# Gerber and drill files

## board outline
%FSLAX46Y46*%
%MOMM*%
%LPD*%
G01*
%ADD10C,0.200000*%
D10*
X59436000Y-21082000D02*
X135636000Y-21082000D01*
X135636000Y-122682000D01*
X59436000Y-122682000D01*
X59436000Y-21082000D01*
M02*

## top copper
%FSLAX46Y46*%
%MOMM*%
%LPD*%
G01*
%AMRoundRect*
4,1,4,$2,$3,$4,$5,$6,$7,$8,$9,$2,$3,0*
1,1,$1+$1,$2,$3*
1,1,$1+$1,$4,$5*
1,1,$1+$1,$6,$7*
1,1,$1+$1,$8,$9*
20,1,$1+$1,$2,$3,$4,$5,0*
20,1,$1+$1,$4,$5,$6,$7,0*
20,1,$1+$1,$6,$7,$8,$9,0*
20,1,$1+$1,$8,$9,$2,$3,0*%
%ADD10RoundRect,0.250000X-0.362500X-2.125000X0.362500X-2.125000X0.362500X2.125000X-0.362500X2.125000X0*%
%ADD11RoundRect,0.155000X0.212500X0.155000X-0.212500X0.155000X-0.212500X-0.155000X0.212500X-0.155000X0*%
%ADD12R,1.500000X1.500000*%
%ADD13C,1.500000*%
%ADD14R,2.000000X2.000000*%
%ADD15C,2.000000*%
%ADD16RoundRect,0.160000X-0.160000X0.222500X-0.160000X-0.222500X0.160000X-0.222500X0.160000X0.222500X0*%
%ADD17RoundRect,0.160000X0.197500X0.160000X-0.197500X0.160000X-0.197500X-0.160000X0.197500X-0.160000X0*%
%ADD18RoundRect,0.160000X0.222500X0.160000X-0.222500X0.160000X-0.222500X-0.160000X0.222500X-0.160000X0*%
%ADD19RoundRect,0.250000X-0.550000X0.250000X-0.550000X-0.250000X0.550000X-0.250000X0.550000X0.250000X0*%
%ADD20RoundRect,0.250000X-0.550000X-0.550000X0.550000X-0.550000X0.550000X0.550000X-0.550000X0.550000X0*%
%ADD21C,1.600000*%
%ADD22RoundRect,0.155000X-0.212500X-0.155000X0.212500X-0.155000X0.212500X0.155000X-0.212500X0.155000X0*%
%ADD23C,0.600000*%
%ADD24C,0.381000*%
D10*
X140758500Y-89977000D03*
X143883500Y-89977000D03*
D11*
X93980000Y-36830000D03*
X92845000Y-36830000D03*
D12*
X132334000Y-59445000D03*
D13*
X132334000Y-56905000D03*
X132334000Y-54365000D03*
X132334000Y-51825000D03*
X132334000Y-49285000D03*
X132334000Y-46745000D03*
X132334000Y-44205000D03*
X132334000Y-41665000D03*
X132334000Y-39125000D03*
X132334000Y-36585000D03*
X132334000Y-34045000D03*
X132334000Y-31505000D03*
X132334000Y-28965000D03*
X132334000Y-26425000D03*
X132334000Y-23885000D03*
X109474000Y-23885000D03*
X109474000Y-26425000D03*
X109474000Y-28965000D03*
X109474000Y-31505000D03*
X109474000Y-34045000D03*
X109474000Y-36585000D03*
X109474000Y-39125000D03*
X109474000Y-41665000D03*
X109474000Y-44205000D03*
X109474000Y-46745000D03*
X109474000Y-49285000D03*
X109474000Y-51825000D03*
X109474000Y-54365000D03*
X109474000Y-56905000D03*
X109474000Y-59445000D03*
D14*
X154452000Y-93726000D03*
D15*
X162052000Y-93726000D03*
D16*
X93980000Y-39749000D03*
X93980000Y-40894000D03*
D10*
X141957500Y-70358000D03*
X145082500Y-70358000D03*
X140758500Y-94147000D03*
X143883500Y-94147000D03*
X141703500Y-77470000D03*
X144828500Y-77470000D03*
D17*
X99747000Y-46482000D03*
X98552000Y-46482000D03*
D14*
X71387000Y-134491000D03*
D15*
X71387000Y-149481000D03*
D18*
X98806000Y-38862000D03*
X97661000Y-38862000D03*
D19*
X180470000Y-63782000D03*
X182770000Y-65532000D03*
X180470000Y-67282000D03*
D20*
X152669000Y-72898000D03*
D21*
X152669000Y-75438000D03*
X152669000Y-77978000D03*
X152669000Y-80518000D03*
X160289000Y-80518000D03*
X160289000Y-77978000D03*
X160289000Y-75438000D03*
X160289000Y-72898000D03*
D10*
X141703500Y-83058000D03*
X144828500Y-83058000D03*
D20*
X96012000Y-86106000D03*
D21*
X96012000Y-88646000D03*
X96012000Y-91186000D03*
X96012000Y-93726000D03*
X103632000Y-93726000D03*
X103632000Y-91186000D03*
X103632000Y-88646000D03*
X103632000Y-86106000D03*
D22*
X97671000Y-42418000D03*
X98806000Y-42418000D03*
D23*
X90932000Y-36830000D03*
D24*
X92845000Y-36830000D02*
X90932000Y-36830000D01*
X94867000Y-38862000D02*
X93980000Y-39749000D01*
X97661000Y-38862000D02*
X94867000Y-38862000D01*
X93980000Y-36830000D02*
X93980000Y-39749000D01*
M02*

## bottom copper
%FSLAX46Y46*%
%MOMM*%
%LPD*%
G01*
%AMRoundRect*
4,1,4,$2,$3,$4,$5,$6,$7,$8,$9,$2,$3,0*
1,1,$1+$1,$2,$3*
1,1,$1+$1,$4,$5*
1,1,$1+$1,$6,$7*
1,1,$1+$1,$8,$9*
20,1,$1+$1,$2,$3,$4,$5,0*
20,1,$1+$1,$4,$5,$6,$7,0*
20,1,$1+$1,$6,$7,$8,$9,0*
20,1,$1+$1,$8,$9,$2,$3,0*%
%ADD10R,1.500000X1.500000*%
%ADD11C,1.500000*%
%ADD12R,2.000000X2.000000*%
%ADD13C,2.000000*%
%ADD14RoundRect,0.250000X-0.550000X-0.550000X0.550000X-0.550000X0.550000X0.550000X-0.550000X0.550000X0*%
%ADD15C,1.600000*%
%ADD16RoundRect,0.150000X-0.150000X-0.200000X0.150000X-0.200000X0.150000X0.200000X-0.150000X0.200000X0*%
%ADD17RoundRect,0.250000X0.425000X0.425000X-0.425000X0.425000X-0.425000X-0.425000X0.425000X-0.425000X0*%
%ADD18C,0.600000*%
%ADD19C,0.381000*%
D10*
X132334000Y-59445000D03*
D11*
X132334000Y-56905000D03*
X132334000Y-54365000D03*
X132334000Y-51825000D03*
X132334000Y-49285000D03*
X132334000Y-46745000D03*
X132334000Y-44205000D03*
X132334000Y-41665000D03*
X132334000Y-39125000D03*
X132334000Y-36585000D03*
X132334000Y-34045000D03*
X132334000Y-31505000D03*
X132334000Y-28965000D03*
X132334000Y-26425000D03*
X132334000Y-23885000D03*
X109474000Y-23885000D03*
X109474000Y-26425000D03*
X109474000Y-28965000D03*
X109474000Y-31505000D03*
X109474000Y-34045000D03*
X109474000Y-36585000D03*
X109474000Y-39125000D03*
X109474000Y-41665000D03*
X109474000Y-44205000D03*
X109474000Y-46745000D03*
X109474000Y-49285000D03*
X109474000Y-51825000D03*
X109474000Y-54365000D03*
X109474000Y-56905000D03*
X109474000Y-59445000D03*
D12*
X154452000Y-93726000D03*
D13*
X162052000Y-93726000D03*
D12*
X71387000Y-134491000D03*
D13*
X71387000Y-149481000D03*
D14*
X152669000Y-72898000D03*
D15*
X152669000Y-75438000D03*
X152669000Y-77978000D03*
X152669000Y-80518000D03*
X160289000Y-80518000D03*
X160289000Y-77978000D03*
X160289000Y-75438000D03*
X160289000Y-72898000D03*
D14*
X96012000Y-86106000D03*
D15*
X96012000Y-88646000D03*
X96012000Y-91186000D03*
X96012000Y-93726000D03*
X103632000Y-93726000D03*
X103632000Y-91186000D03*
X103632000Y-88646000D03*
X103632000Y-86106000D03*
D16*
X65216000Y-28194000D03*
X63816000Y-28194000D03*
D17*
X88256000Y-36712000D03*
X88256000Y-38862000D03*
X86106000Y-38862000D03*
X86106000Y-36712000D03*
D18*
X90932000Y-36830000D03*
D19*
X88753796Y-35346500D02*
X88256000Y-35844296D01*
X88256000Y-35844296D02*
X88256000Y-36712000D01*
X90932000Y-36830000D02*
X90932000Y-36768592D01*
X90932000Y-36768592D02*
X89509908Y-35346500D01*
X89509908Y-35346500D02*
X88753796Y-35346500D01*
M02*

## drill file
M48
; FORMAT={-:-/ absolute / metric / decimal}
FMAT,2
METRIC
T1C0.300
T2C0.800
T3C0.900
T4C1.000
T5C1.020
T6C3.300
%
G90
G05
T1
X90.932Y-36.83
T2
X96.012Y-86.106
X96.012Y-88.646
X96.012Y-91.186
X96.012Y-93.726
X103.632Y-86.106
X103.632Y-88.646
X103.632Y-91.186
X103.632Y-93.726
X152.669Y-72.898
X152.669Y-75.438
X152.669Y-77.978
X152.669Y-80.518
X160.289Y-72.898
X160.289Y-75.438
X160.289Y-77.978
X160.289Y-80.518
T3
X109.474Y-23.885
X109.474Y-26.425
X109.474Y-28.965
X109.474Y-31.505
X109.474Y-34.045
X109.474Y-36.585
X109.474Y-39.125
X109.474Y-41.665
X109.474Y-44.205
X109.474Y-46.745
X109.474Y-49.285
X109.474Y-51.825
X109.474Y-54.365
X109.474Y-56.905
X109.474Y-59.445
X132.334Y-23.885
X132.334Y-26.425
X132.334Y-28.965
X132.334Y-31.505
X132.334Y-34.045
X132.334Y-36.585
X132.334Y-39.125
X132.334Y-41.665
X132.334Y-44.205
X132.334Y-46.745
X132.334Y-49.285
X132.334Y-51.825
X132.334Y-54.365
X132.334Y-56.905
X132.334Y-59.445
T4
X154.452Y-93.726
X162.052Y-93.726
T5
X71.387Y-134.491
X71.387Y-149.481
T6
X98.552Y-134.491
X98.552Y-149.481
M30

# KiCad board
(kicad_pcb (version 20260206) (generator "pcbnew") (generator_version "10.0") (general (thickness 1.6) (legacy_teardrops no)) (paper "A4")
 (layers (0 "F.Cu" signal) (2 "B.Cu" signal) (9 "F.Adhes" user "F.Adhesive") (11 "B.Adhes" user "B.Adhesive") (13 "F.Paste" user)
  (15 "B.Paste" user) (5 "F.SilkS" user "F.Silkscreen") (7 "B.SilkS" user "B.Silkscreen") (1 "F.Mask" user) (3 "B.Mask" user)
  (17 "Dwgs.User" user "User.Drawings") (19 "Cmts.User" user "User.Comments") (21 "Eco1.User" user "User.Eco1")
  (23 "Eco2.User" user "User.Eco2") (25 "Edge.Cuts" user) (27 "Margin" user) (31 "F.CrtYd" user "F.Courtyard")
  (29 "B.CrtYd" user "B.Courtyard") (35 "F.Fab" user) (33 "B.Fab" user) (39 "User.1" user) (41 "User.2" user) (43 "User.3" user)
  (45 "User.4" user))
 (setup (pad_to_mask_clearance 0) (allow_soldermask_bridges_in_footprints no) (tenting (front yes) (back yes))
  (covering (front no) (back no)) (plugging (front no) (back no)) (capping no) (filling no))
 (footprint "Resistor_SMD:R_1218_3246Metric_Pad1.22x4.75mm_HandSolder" (layer "F.Cu") (at 142.321 89.977)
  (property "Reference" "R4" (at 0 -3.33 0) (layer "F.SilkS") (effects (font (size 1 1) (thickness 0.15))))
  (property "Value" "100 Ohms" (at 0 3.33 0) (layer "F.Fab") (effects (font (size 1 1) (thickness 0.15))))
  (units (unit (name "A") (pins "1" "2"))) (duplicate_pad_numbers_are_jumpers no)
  (pad "1" smd roundrect (at -1.5625 0) (size 1.225 4.75) (layers "F.Cu" "F.Mask" "F.Paste") (roundrect_rratio 0.204082) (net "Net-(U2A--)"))
  (pad "2" smd roundrect (at 1.5625 0) (size 1.225 4.75) (layers "F.Cu" "F.Mask" "F.Paste") (roundrect_rratio 0.204082)
   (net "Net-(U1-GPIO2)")))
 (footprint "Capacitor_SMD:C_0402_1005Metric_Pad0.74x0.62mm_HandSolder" (layer "F.Cu") (at 93.4125 36.83 180)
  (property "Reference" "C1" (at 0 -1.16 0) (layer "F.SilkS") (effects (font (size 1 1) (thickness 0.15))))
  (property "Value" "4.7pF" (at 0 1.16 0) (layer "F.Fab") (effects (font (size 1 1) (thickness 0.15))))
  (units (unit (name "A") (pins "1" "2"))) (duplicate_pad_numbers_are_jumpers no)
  (pad "1" smd roundrect (at -0.5675 0 180) (size 0.735 0.62) (layers "F.Cu" "F.Mask" "F.Paste") (roundrect_rratio 0.25) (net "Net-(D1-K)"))
  (pad "2" smd roundrect (at 0.5675 0 180) (size 0.735 0.62) (layers "F.Cu" "F.Mask" "F.Paste") (roundrect_rratio 0.25) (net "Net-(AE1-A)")))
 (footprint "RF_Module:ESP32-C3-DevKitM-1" (layer "F.Cu") (at 132.334 59.445 180)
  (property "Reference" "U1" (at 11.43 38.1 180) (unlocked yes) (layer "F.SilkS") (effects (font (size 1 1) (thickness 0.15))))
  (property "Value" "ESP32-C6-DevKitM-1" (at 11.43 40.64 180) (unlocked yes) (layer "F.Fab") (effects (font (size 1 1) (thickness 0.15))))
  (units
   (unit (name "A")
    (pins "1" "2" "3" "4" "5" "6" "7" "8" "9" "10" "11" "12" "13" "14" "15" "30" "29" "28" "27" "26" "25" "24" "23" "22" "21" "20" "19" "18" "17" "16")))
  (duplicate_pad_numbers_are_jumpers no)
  (pad "1" thru_hole rect (at 0 0 180) (size 1.5 1.5) (drill 0.9) (layers "*.Cu" "*.Mask") (remove_unused_layers yes) (keep_end_layers yes)
   (zone_layer_connections) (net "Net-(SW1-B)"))
  (pad "2" thru_hole circle (at 0 2.54 180) (size 1.5 1.5) (drill 0.9) (layers "*.Cu" "*.Mask") (remove_unused_layers yes)
   (keep_end_layers yes) (zone_layer_connections) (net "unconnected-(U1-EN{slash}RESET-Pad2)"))
  (pad "3" thru_hole circle (at 0 5.08 180) (size 1.5 1.5) (drill 0.9) (layers "*.Cu" "*.Mask") (remove_unused_layers yes)
   (keep_end_layers yes) (zone_layer_connections) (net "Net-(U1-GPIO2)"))
  (pad "4" thru_hole circle (at 0 7.62 180) (size 1.5 1.5) (drill 0.9) (layers "*.Cu" "*.Mask") (remove_unused_layers yes)
   (keep_end_layers yes) (zone_layer_connections) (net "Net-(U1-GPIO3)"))
  (pad "5" thru_hole circle (at 0 10.16 180) (size 1.5 1.5) (drill 0.9) (layers "*.Cu" "*.Mask") (remove_unused_layers yes)
   (keep_end_layers yes) (zone_layer_connections) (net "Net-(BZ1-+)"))
  (pad "6" thru_hole circle (at 0 12.7 180) (size 1.5 1.5) (drill 0.9) (layers "*.Cu" "*.Mask") (remove_unused_layers yes)
   (keep_end_layers yes) (zone_layer_connections) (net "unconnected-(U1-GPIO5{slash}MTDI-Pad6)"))
  (pad "7" thru_hole circle (at 0 15.24 180) (size 1.5 1.5) (drill 0.9) (layers "*.Cu" "*.Mask") (remove_unused_layers yes)
   (keep_end_layers yes) (zone_layer_connections) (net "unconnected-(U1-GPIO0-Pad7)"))
  (pad "8" thru_hole circle (at 0 17.78 180) (size 1.5 1.5) (drill 0.9) (layers "*.Cu" "*.Mask") (remove_unused_layers yes)
   (keep_end_layers yes) (zone_layer_connections) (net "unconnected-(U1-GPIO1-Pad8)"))
  (pad "9" thru_hole circle (at 0 20.32 180) (size 1.5 1.5) (drill 0.9) (layers "*.Cu" "*.Mask") (remove_unused_layers yes)
   (keep_end_layers yes) (zone_layer_connections) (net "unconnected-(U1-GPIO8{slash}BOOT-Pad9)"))
  (pad "10" thru_hole circle (at 0 22.86 180) (size 1.5 1.5) (drill 0.9) (layers "*.Cu" "*.Mask") (remove_unused_layers yes)
   (keep_end_layers yes) (zone_layer_connections) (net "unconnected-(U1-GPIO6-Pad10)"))
  (pad "11" thru_hole circle (at 0 25.4 180) (size 1.5 1.5) (drill 0.9) (layers "*.Cu" "*.Mask") (remove_unused_layers yes)
   (keep_end_layers yes) (zone_layer_connections) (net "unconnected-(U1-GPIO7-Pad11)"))
  (pad "12" thru_hole circle (at 0 27.94 180) (size 1.5 1.5) (drill 0.9) (layers "*.Cu" "*.Mask") (remove_unused_layers yes)
   (keep_end_layers yes) (zone_layer_connections) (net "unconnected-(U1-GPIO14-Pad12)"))
  (pad "13" thru_hole circle (at 0 30.48 180) (size 1.5 1.5) (drill 0.9) (layers "*.Cu" "*.Mask") (remove_unused_layers yes)
   (keep_end_layers yes) (zone_layer_connections) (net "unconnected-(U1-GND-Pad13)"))
  (pad "14" thru_hole circle (at 0 33.02 180) (size 1.5 1.5) (drill 0.9) (layers "*.Cu" "*.Mask") (remove_unused_layers yes)
   (keep_end_layers yes) (zone_layer_connections) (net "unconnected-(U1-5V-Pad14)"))
  (pad "15" thru_hole circle (at 0 35.56 180) (size 1.5 1.5) (drill 0.9) (layers "*.Cu" "*.Mask") (remove_unused_layers yes)
   (keep_end_layers yes) (zone_layer_connections) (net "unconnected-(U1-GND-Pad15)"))
  (pad "16" thru_hole circle (at 22.86 35.56 180) (size 1.5 1.5) (drill 0.9) (layers "*.Cu" "*.Mask") (remove_unused_layers yes)
   (keep_end_layers yes) (zone_layer_connections) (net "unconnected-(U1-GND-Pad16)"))
  (pad "17" thru_hole circle (at 22.86 33.02 180) (size 1.5 1.5) (drill 0.9) (layers "*.Cu" "*.Mask") (remove_unused_layers yes)
   (keep_end_layers yes) (zone_layer_connections) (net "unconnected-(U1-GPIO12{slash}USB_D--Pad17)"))
  (pad "18" thru_hole circle (at 22.86 30.48 180) (size 1.5 1.5) (drill 0.9) (layers "*.Cu" "*.Mask") (remove_unused_layers yes)
   (keep_end_layers yes) (zone_layer_connections) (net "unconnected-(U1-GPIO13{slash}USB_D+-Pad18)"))
  (pad "19" thru_hole circle (at 22.86 27.94 180) (size 1.5 1.5) (drill 0.9) (layers "*.Cu" "*.Mask") (remove_unused_layers yes)
   (keep_end_layers yes) (zone_layer_connections) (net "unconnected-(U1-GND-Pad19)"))
  (pad "20" thru_hole circle (at 22.86 25.4 180) (size 1.5 1.5) (drill 0.9) (layers "*.Cu" "*.Mask") (remove_unused_layers yes)
   (keep_end_layers yes) (zone_layer_connections) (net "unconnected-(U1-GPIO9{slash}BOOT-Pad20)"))
  (pad "21" thru_hole circle (at 22.86 22.86 180) (size 1.5 1.5) (drill 0.9) (layers "*.Cu" "*.Mask") (remove_unused_layers yes)
   (keep_end_layers yes) (zone_layer_connections) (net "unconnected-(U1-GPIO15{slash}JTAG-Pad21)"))
  (pad "22" thru_hole circle (at 22.86 20.32 180) (size 1.5 1.5) (drill 0.9) (layers "*.Cu" "*.Mask") (remove_unused_layers yes)
   (keep_end_layers yes) (zone_layer_connections) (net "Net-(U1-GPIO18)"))
  (pad "23" thru_hole circle (at 22.86 17.78 180) (size 1.5 1.5) (drill 0.9) (layers "*.Cu" "*.Mask") (remove_unused_layers yes)
   (keep_end_layers yes) (zone_layer_connections) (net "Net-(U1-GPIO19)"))
  (pad "24" thru_hole circle (at 22.86 15.24 180) (size 1.5 1.5) (drill 0.9) (layers "*.Cu" "*.Mask") (remove_unused_layers yes)
   (keep_end_layers yes) (zone_layer_connections) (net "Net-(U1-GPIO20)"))
  (pad "25" thru_hole circle (at 22.86 12.7 180) (size 1.5 1.5) (drill 0.9) (layers "*.Cu" "*.Mask") (remove_unused_layers yes)
   (keep_end_layers yes) (zone_layer_connections) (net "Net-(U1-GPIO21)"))
  (pad "26" thru_hole circle (at 22.86 10.16 180) (size 1.5 1.5) (drill 0.9) (layers "*.Cu" "*.Mask") (remove_unused_layers yes)
   (keep_end_layers yes) (zone_layer_connections) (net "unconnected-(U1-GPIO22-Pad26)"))
  (pad "27" thru_hole circle (at 22.86 7.62 180) (size 1.5 1.5) (drill 0.9) (layers "*.Cu" "*.Mask") (remove_unused_layers yes)
   (keep_end_layers yes) (zone_layer_connections) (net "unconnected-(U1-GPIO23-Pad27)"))
  (pad "28" thru_hole circle (at 22.86 5.08 180) (size 1.5 1.5) (drill 0.9) (layers "*.Cu" "*.Mask") (remove_unused_layers yes)
   (keep_end_layers yes) (zone_layer_connections) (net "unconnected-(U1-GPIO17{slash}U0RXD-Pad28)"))
  (pad "29" thru_hole circle (at 22.86 2.54 180) (size 1.5 1.5) (drill 0.9) (layers "*.Cu" "*.Mask") (remove_unused_layers yes)
   (keep_end_layers yes) (zone_layer_connections) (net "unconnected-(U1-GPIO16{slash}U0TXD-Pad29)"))
  (pad "30" thru_hole circle (at 22.86 0 180) (size 1.5 1.5) (drill 0.9) (layers "*.Cu" "*.Mask") (remove_unused_layers yes)
   (keep_end_layers yes) (zone_layer_connections) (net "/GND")))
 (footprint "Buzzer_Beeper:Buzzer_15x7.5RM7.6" (layer "F.Cu") (at 154.452 93.726)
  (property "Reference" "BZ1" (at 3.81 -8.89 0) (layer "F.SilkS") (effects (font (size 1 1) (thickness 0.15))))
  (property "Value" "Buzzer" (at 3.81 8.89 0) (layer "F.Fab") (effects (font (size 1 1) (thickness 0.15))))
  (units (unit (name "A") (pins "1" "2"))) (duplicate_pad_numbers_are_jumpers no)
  (pad "1" thru_hole rect (at 0 0) (size 2 2) (drill 1) (layers "*.Cu" "*.Mask") (remove_unused_layers no) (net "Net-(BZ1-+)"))
  (pad "2" thru_hole circle (at 7.6 0) (size 2 2) (drill 1) (layers "*.Cu" "*.Mask") (remove_unused_layers no) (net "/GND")))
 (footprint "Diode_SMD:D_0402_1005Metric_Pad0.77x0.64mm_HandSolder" (layer "F.Cu") (at 93.98 40.3215 -90)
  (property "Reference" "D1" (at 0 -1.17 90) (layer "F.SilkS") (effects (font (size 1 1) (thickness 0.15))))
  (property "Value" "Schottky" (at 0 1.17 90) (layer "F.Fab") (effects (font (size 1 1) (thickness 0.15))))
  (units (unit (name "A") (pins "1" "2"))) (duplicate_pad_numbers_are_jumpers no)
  (pad "1" smd roundrect (at -0.5725 0 270) (size 0.765 0.64) (layers "F.Cu" "F.Mask" "F.Paste") (roundrect_rratio 0.25) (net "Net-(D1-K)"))
  (pad "2" smd roundrect (at 0.5725 0 270) (size 0.765 0.64) (layers "F.Cu" "F.Mask" "F.Paste") (roundrect_rratio 0.25) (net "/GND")))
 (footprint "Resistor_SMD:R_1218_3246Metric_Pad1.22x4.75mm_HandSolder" (layer "F.Cu") (at 143.52 70.358)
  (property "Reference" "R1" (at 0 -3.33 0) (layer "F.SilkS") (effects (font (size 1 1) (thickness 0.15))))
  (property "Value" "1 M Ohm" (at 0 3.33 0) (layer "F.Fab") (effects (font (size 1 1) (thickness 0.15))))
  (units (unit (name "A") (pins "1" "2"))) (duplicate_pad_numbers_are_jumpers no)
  (pad "1" smd roundrect (at -1.5625 0) (size 1.225 4.75) (layers "F.Cu" "F.Mask" "F.Paste") (roundrect_rratio 0.204082) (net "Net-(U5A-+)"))
  (pad "2" smd roundrect (at 1.5625 0) (size 1.225 4.75) (layers "F.Cu" "F.Mask" "F.Paste") (roundrect_rratio 0.204082) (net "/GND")))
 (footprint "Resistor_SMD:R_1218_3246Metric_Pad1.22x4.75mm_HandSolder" (layer "F.Cu") (at 142.321 94.147)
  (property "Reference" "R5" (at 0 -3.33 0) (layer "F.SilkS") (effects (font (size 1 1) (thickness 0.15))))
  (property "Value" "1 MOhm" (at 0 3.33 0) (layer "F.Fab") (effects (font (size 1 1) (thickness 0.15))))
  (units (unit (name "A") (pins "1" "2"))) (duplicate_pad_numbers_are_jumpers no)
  (pad "1" smd roundrect (at -1.5625 0) (size 1.225 4.75) (layers "F.Cu" "F.Mask" "F.Paste") (roundrect_rratio 0.204082) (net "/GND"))
  (pad "2" smd roundrect (at 1.5625 0) (size 1.225 4.75) (layers "F.Cu" "F.Mask" "F.Paste") (roundrect_rratio 0.204082) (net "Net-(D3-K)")))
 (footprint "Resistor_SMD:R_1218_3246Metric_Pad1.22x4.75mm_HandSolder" (layer "F.Cu") (at 143.266 77.47)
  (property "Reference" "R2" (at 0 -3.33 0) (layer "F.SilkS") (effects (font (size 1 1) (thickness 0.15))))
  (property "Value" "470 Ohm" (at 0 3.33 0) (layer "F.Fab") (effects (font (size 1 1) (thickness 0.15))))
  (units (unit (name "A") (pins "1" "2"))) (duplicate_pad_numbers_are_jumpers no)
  (pad "1" smd roundrect (at -1.5625 0) (size 1.225 4.75) (layers "F.Cu" "F.Mask" "F.Paste") (roundrect_rratio 0.204082)
   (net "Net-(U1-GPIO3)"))
  (pad "2" smd roundrect (at 1.5625 0) (size 1.225 4.75) (layers "F.Cu" "F.Mask" "F.Paste") (roundrect_rratio 0.204082)
   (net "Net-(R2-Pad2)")))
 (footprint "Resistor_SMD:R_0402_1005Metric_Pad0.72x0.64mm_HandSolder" (layer "F.Cu") (at 99.1495 46.482 180)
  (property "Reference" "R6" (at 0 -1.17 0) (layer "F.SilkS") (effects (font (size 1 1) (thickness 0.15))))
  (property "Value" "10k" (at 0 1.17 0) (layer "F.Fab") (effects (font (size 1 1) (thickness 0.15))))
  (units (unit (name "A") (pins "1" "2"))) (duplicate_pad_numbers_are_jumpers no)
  (pad "1" smd roundrect (at -0.5975 0 180) (size 0.715 0.64) (layers "F.Cu" "F.Mask" "F.Paste") (roundrect_rratio 0.25) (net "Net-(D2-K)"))
  (pad "2" smd roundrect (at 0.5975 0 180) (size 0.715 0.64) (layers "F.Cu" "F.Mask" "F.Paste") (roundrect_rratio 0.25) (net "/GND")))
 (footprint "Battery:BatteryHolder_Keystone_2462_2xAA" (layer "F.Cu") (at 71.387 134.491)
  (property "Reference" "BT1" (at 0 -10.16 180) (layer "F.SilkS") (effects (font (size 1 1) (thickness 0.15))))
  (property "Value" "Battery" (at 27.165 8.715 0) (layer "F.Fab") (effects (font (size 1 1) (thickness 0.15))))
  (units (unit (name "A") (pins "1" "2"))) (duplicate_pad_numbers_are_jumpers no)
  (pad "" np_thru_hole circle (at 27.165 0) (size 3.3 3.3) (drill 3.3) (layers "*.Cu" "*.Mask"))
  (pad "" np_thru_hole circle (at 27.165 14.99) (size 3.3 3.3) (drill 3.3) (layers "*.Cu" "*.Mask"))
  (pad "1" thru_hole rect (at 0 0) (size 2 2) (drill 1.02) (layers "*.Cu" "*.Mask") (remove_unused_layers no) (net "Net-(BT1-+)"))
  (pad "2" thru_hole circle (at 0 14.99) (size 2 2) (drill 1.02) (layers "*.Cu" "*.Mask") (remove_unused_layers no) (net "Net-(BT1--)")))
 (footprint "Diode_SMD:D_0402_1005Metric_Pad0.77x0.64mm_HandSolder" (layer "F.Cu") (at 98.2335 38.862 180)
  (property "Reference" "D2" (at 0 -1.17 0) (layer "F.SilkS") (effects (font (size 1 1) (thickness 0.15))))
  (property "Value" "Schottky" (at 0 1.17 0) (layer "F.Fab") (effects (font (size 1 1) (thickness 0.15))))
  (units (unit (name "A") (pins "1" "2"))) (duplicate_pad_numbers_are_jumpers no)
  (pad "1" smd roundrect (at -0.5725 0 180) (size 0.765 0.64) (layers "F.Cu" "F.Mask" "F.Paste") (roundrect_rratio 0.25) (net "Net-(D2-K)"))
  (pad "2" smd roundrect (at 0.5725 0 180) (size 0.765 0.64) (layers "F.Cu" "F.Mask" "F.Paste") (roundrect_rratio 0.25) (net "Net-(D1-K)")))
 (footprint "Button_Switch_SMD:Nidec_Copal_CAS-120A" (layer "F.Cu") (at 181.62 65.532)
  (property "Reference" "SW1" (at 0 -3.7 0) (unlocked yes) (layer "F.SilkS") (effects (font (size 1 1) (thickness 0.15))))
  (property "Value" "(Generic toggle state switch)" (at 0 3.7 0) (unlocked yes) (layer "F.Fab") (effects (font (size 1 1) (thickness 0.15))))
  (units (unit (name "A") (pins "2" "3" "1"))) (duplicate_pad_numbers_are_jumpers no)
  (pad "1" smd roundrect (at -1.15 -1.75 270) (size 1 1.6) (layers "F.Cu" "F.Mask" "F.Paste") (roundrect_rratio 0.25) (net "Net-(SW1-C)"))
  (pad "2" smd roundrect (at 1.15 0 270) (size 1 1.6) (layers "F.Cu" "F.Mask" "F.Paste") (roundrect_rratio 0.25) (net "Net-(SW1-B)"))
  (pad "3" smd roundrect (at -1.15 1.75 270) (size 1 1.6) (layers "F.Cu" "F.Mask" "F.Paste") (roundrect_rratio 0.25) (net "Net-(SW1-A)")))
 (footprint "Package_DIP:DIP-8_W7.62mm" (layer "F.Cu") (at 152.669 72.898)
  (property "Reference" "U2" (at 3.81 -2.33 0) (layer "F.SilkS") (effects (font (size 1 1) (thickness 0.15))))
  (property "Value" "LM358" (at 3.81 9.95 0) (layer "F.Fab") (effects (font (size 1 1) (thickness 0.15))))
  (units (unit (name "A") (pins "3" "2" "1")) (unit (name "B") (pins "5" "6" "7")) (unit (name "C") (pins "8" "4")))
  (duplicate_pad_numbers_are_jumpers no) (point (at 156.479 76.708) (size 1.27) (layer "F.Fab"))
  (pad "1" thru_hole roundrect (at 0 0) (size 1.6 1.6) (drill 0.8) (layers "*.Cu" "*.Mask") (remove_unused_layers no)
   (roundrect_rratio 0.15625) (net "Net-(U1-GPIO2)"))
  (pad "2" thru_hole circle (at 0 2.54) (size 1.6 1.6) (drill 0.8) (layers "*.Cu" "*.Mask") (remove_unused_layers no) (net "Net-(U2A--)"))
  (pad "3" thru_hole circle (at 0 5.08) (size 1.6 1.6) (drill 0.8) (layers "*.Cu" "*.Mask") (remove_unused_layers no) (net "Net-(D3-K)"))
  (pad "4" thru_hole circle (at 0 7.62) (size 1.6 1.6) (drill 0.8) (layers "*.Cu" "*.Mask") (remove_unused_layers no) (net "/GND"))
  (pad "5" thru_hole circle (at 7.62 7.62) (size 1.6 1.6) (drill 0.8) (layers "*.Cu" "*.Mask") (remove_unused_layers no))
  (pad "6" thru_hole circle (at 7.62 5.08) (size 1.6 1.6) (drill 0.8) (layers "*.Cu" "*.Mask") (remove_unused_layers no))
  (pad "7" thru_hole circle (at 7.62 2.54) (size 1.6 1.6) (drill 0.8) (layers "*.Cu" "*.Mask") (remove_unused_layers no))
  (pad "8" thru_hole circle (at 7.62 0) (size 1.6 1.6) (drill 0.8) (layers "*.Cu" "*.Mask") (remove_unused_layers no) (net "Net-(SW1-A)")))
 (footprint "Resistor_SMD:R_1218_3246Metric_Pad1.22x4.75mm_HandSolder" (layer "F.Cu") (at 143.266 83.058)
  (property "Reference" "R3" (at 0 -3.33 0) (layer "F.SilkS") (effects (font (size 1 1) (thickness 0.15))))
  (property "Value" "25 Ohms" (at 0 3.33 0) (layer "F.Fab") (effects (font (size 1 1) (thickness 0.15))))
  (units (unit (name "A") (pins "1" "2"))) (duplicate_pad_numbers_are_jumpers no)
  (pad "1" smd roundrect (at -1.5625 0) (size 1.225 4.75) (layers "F.Cu" "F.Mask" "F.Paste") (roundrect_rratio 0.204082) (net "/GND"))
  (pad "2" smd roundrect (at 1.5625 0) (size 1.225 4.75) (layers "F.Cu" "F.Mask" "F.Paste") (roundrect_rratio 0.204082) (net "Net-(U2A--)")))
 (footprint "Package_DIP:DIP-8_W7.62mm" (layer "F.Cu") (at 96.012 86.106)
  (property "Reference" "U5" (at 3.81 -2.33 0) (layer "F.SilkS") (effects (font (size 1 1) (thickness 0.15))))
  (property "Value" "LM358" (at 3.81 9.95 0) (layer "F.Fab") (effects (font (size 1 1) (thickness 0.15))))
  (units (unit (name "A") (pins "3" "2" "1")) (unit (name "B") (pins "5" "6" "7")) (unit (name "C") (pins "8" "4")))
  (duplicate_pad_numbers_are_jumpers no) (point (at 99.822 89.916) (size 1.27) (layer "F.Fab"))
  (pad "1" thru_hole roundrect (at 0 0) (size 1.6 1.6) (drill 0.8) (layers "*.Cu" "*.Mask") (remove_unused_layers no)
   (roundrect_rratio 0.15625) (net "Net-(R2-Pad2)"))
  (pad "2" thru_hole circle (at 0 2.54) (size 1.6 1.6) (drill 0.8) (layers "*.Cu" "*.Mask") (remove_unused_layers no) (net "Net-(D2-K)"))
  (pad "3" thru_hole circle (at 0 5.08) (size 1.6 1.6) (drill 0.8) (layers "*.Cu" "*.Mask") (remove_unused_layers no) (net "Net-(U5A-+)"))
  (pad "4" thru_hole circle (at 0 7.62) (size 1.6 1.6) (drill 0.8) (layers "*.Cu" "*.Mask") (remove_unused_layers no) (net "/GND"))
  (pad "5" thru_hole circle (at 7.62 7.62) (size 1.6 1.6) (drill 0.8) (layers "*.Cu" "*.Mask") (remove_unused_layers no))
  (pad "6" thru_hole circle (at 7.62 5.08) (size 1.6 1.6) (drill 0.8) (layers "*.Cu" "*.Mask") (remove_unused_layers no))
  (pad "7" thru_hole circle (at 7.62 2.54) (size 1.6 1.6) (drill 0.8) (layers "*.Cu" "*.Mask") (remove_unused_layers no))
  (pad "8" thru_hole circle (at 7.62 0) (size 1.6 1.6) (drill 0.8) (layers "*.Cu" "*.Mask") (remove_unused_layers no) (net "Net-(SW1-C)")))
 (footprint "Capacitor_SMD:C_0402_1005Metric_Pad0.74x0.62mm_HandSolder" (layer "F.Cu") (at 98.2385 42.418)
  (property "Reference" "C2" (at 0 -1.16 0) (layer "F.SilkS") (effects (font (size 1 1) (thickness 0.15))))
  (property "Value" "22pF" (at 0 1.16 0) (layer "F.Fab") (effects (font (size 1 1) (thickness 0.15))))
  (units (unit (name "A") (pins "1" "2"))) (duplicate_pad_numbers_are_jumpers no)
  (pad "1" smd roundrect (at -0.5675 0) (size 0.735 0.62) (layers "F.Cu" "F.Mask" "F.Paste") (roundrect_rratio 0.25) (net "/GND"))
  (pad "2" smd roundrect (at 0.5675 0) (size 0.735 0.62) (layers "F.Cu" "F.Mask" "F.Paste") (roundrect_rratio 0.25) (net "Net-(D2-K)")))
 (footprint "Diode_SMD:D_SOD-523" (layer "B.Cu") (at 64.516 28.194 180)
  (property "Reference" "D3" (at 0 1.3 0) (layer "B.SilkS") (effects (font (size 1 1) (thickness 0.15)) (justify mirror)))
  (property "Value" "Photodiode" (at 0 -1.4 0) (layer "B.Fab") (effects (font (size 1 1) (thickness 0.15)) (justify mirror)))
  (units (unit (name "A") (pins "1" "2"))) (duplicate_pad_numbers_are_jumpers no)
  (pad "1" smd roundrect (at -0.7 0) (size 0.6 0.7) (layers "B.Cu" "B.Mask" "B.Paste") (roundrect_rratio 0.25) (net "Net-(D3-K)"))
  (pad "2" smd roundrect (at 0.7 0) (size 0.6 0.7) (layers "B.Cu" "B.Mask" "B.Paste") (roundrect_rratio 0.25) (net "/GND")))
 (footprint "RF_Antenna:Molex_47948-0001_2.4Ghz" (layer "B.Cu") (at 87.181 37.787 180)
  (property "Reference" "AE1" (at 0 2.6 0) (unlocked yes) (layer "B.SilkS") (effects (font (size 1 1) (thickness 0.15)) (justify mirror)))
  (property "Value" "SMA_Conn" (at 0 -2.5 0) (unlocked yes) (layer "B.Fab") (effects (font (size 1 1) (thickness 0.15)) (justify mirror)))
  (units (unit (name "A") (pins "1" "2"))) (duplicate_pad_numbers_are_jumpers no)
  (pad "1" smd roundrect (at -1.075 1.075 180) (size 1.35 1.35) (layers "B.Cu" "B.Mask" "B.Paste") (roundrect_rratio 0.1851851852)
   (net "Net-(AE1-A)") (thermal_bridge_angle 45))
  (pad "MP" smd roundrect (at -1.075 -1.075 180) (size 1.35 1.35) (layers "B.Cu" "B.Mask" "B.Paste") (roundrect_rratio 0.1851851852)
   (thermal_bridge_angle 45))
  (pad "MP" smd roundrect (at 1.075 -1.075 180) (size 1.35 1.35) (layers "B.Cu" "B.Mask" "B.Paste") (roundrect_rratio 0.1851851852)
   (thermal_bridge_angle 45))
  (pad "MP" smd roundrect (at 1.075 1.075 180) (size 1.35 1.35) (layers "B.Cu" "B.Mask" "B.Paste") (roundrect_rratio 0.1851851852)
   (thermal_bridge_angle 45))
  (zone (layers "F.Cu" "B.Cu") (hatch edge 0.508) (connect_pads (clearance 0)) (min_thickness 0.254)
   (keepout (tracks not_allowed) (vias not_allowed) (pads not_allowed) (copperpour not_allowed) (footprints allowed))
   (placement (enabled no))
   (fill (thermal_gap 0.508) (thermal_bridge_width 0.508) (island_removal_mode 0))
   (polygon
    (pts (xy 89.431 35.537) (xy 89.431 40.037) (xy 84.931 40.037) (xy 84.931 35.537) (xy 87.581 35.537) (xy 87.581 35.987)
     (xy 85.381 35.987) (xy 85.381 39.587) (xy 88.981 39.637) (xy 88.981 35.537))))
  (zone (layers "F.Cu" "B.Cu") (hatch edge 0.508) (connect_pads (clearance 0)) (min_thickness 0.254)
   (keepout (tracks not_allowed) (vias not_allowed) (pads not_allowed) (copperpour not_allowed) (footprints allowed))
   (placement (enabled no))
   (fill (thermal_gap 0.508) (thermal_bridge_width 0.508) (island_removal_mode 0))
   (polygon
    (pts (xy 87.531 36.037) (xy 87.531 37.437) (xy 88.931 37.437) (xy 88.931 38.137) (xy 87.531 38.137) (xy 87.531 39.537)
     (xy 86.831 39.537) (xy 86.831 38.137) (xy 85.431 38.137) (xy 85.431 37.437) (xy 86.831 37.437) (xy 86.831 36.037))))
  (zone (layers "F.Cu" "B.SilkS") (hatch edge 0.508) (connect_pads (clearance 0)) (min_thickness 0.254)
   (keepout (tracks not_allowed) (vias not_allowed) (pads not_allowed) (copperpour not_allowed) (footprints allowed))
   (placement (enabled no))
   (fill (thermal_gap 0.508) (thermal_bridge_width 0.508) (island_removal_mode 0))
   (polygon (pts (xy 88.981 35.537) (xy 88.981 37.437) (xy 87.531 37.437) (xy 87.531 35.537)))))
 (gr_rect (start 59.436 21.082) (end 135.636 122.682) (stroke (width 0.2) (type solid)) (fill no) (layer "Edge.Cuts"))
 (segment (start 92.845 36.83) (end 90.932 36.83) (width 0.381) (layer "F.Cu") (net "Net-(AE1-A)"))
 (via (at 90.932 36.83) (size 0.6) (drill 0.3) (layers "F.Cu" "B.Cu") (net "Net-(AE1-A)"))
 (segment (start 88.753796 35.3465) (end 88.256 35.844296) (width 0.381) (layer "B.Cu") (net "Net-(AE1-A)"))
 (segment (start 88.256 35.844296) (end 88.256 36.712) (width 0.381) (layer "B.Cu") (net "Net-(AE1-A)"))
 (segment (start 90.932 36.83) (end 90.932 36.768592) (width 0.381) (layer "B.Cu") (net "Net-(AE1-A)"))
 (segment (start 90.932 36.768592) (end 89.509908 35.3465) (width 0.381) (layer "B.Cu") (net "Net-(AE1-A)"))
 (segment (start 89.509908 35.3465) (end 88.753796 35.3465) (width 0.381) (layer "B.Cu") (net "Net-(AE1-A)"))
 (segment (start 94.867 38.862) (end 93.98 39.749) (width 0.381) (layer "F.Cu") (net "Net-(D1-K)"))
 (segment (start 97.661 38.862) (end 94.867 38.862) (width 0.381) (layer "F.Cu") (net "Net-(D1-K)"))
 (segment (start 93.98 36.83) (end 93.98 39.749) (width 0.381) (layer "F.Cu") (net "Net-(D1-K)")))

